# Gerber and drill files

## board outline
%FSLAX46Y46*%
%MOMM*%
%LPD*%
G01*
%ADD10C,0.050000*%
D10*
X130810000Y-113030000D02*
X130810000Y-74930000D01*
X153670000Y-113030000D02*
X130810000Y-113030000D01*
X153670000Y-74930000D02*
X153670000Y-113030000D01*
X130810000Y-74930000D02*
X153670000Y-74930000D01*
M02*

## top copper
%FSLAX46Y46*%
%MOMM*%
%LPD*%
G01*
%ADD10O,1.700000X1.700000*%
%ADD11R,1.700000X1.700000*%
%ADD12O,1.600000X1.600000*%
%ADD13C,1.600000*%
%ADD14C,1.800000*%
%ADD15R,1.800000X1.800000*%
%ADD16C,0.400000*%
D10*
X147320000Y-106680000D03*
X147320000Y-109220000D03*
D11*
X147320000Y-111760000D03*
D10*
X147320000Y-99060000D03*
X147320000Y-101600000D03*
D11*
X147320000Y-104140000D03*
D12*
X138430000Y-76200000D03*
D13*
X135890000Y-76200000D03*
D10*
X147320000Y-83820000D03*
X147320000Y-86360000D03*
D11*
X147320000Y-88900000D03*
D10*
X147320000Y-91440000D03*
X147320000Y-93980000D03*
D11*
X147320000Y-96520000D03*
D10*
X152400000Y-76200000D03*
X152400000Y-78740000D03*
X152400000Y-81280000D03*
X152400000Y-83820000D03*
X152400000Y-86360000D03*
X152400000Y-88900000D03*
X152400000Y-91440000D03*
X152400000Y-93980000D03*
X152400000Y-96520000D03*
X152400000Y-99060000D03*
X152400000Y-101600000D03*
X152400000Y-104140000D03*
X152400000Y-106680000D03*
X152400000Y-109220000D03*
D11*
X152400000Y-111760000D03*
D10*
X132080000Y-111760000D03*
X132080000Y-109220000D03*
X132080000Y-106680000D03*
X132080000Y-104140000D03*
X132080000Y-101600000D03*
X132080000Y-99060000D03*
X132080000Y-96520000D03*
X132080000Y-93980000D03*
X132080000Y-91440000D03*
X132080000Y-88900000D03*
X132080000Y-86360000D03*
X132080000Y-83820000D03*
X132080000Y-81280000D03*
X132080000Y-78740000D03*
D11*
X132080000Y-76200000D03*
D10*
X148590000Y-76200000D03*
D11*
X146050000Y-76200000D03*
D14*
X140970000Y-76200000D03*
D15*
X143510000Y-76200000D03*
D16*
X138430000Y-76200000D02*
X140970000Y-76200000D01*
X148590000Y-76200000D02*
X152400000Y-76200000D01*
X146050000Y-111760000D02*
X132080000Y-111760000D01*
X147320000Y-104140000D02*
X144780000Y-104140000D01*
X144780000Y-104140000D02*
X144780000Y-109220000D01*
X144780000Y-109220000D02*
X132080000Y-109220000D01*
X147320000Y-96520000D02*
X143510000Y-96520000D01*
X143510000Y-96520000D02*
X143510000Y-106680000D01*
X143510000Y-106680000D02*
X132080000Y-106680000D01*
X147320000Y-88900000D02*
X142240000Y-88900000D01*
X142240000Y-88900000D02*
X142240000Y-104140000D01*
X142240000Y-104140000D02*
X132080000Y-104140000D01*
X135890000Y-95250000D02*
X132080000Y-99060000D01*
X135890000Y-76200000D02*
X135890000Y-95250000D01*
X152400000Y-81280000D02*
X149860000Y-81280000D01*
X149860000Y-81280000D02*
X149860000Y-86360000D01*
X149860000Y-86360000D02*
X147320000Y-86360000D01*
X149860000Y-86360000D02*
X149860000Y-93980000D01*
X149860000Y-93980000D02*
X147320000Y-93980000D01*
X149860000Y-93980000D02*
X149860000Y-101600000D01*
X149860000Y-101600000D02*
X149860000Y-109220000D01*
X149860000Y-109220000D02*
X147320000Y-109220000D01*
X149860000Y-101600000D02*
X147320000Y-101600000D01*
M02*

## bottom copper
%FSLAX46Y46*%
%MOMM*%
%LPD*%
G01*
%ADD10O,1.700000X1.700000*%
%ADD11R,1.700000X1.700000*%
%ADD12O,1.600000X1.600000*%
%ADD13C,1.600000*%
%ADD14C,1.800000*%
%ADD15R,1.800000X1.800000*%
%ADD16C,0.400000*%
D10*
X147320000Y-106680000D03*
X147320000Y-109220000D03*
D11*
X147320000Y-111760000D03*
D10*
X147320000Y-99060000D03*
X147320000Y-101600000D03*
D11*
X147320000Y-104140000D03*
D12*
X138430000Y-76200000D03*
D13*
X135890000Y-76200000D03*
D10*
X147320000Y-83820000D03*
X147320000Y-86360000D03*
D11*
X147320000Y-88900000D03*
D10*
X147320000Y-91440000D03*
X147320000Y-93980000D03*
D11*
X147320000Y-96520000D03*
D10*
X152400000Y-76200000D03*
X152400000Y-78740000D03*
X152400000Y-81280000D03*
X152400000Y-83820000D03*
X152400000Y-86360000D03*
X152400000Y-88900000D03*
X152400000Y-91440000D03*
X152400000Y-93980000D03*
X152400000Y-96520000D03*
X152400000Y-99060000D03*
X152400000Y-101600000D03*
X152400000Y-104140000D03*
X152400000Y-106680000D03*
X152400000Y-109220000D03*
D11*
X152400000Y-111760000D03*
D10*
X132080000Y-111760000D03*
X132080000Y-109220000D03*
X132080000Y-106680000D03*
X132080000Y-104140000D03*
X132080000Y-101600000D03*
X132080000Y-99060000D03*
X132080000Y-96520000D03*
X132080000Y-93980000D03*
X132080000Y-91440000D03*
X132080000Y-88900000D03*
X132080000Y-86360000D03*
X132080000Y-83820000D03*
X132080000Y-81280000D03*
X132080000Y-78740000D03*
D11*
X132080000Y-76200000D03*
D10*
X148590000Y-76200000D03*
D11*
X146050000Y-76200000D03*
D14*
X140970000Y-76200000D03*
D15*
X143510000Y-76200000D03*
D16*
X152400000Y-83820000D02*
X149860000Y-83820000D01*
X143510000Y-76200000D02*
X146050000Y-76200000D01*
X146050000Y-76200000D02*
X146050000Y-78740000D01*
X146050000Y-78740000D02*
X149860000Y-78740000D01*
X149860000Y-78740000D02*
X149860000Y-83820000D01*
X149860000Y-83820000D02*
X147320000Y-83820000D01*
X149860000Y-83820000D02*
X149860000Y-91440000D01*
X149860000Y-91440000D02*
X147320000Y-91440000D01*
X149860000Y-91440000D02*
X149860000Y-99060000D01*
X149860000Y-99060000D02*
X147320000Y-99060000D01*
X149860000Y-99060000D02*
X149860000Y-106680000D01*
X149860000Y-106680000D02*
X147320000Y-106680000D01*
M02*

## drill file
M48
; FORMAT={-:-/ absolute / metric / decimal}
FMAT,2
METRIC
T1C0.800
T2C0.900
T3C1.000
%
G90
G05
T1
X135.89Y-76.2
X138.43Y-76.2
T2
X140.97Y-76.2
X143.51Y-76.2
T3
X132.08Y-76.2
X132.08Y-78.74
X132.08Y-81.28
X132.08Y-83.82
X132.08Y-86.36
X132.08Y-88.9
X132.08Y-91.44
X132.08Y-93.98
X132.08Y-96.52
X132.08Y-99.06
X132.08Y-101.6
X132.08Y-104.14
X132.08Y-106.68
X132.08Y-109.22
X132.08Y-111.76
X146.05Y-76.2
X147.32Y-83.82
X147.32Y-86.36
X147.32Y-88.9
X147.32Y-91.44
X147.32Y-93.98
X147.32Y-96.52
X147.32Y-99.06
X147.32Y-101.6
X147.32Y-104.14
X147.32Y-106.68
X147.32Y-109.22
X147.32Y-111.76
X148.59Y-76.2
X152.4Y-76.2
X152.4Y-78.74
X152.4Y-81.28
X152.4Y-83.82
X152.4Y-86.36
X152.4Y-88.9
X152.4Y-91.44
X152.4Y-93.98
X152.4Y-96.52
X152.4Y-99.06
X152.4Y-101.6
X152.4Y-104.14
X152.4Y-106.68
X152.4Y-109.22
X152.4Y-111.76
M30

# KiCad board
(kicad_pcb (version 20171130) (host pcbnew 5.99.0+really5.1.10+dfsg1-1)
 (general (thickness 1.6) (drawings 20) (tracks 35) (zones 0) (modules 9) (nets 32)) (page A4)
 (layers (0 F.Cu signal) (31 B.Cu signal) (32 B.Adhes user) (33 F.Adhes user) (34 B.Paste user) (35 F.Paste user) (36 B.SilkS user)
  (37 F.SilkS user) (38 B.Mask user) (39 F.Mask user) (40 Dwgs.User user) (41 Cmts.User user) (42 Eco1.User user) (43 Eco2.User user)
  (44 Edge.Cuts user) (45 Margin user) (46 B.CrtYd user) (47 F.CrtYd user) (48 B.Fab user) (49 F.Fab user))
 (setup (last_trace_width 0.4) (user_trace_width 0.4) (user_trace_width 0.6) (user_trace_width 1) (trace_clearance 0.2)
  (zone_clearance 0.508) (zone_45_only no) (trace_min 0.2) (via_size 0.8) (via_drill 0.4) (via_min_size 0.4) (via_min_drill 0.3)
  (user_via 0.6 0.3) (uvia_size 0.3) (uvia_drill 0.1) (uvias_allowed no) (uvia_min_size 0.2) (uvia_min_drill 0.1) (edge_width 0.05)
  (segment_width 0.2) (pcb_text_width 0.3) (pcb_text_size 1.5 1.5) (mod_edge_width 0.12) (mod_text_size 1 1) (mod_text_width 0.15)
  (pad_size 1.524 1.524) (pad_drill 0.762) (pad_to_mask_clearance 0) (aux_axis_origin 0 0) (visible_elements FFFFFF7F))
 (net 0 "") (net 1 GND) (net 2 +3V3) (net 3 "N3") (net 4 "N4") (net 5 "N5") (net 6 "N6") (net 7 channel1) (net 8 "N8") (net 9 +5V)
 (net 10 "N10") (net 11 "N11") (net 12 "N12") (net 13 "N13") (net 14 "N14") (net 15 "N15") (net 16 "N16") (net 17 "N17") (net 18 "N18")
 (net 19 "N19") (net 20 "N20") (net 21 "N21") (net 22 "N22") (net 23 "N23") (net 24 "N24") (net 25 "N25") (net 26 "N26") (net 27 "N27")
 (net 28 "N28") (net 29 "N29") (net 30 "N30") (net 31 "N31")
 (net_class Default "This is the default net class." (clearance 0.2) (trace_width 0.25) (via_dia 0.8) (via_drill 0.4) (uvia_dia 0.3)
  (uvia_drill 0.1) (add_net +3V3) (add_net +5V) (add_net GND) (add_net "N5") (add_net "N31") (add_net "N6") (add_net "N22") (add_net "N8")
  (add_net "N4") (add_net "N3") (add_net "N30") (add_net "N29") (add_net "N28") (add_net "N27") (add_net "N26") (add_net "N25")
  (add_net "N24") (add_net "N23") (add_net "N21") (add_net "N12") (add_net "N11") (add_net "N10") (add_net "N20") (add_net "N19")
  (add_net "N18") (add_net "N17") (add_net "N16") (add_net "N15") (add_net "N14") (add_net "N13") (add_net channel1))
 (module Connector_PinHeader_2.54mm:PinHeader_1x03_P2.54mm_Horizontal (layer F.Cu) (at 147.32 111.76 180)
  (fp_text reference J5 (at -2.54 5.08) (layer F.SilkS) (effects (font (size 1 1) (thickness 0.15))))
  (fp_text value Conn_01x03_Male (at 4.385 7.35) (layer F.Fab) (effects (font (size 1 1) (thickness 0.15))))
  (pad 3 thru_hole oval (at 0 5.08 180) (size 1.7 1.7) (drill 1) (layers *.Cu *.Mask) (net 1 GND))
  (pad 2 thru_hole oval (at 0 2.54 180) (size 1.7 1.7) (drill 1) (layers *.Cu *.Mask) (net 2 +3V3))
  (pad 1 thru_hole rect (at 0 0 180) (size 1.7 1.7) (drill 1) (layers *.Cu *.Mask) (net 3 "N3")))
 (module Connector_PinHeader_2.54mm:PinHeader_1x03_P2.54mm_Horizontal (layer F.Cu) (at 147.32 104.14 180)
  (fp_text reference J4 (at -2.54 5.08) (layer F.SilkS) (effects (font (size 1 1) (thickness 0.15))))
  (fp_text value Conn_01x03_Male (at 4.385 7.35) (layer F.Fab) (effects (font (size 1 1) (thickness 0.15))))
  (pad 3 thru_hole oval (at 0 5.08 180) (size 1.7 1.7) (drill 1) (layers *.Cu *.Mask) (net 1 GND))
  (pad 2 thru_hole oval (at 0 2.54 180) (size 1.7 1.7) (drill 1) (layers *.Cu *.Mask) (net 2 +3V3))
  (pad 1 thru_hole rect (at 0 0 180) (size 1.7 1.7) (drill 1) (layers *.Cu *.Mask) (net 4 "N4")))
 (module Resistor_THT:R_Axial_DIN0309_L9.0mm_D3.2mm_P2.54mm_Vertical (layer F.Cu) (at 135.89 76.2)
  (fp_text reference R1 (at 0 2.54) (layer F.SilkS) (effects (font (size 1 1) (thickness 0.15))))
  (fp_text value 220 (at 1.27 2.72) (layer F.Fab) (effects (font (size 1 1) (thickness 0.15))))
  (pad 2 thru_hole oval (at 2.54 0) (size 1.6 1.6) (drill 0.8) (layers *.Cu *.Mask) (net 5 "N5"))
  (pad 1 thru_hole circle (at 0 0) (size 1.6 1.6) (drill 0.8) (layers *.Cu *.Mask) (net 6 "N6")))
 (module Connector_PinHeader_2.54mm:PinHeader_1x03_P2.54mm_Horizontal (layer F.Cu) (at 147.32 88.9 180)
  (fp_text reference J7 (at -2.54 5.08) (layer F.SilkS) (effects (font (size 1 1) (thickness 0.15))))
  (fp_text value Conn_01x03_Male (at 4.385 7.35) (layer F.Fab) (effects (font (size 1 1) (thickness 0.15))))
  (pad 3 thru_hole oval (at 0 5.08 180) (size 1.7 1.7) (drill 1) (layers *.Cu *.Mask) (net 1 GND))
  (pad 2 thru_hole oval (at 0 2.54 180) (size 1.7 1.7) (drill 1) (layers *.Cu *.Mask) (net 2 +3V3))
  (pad 1 thru_hole rect (at 0 0 180) (size 1.7 1.7) (drill 1) (layers *.Cu *.Mask) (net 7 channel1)))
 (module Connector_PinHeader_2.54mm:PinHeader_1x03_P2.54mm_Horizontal (layer F.Cu) (at 147.32 96.52 180)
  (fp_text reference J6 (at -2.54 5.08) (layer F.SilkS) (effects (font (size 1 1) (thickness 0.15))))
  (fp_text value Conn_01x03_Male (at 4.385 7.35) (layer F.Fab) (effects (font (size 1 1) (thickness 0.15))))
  (pad 3 thru_hole oval (at 0 5.08 180) (size 1.7 1.7) (drill 1) (layers *.Cu *.Mask) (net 1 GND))
  (pad 2 thru_hole oval (at 0 2.54 180) (size 1.7 1.7) (drill 1) (layers *.Cu *.Mask) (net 2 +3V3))
  (pad 1 thru_hole rect (at 0 0 180) (size 1.7 1.7) (drill 1) (layers *.Cu *.Mask) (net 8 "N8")))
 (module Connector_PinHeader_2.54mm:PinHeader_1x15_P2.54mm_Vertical (layer F.Cu) (at 152.4 111.76 180)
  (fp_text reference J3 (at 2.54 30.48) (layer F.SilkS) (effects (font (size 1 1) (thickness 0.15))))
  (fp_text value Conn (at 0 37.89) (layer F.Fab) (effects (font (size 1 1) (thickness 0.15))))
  (pad 15 thru_hole oval (at 0 35.56 180) (size 1.7 1.7) (drill 1) (layers *.Cu *.Mask) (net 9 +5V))
  (pad 14 thru_hole oval (at 0 33.02 180) (size 1.7 1.7) (drill 1) (layers *.Cu *.Mask) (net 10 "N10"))
  (pad 13 thru_hole oval (at 0 30.48 180) (size 1.7 1.7) (drill 1) (layers *.Cu *.Mask) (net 2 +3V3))
  (pad 12 thru_hole oval (at 0 27.94 180) (size 1.7 1.7) (drill 1) (layers *.Cu *.Mask) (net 1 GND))
  (pad 11 thru_hole oval (at 0 25.4 180) (size 1.7 1.7) (drill 1) (layers *.Cu *.Mask) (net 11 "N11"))
  (pad 10 thru_hole oval (at 0 22.86 180) (size 1.7 1.7) (drill 1) (layers *.Cu *.Mask) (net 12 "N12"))
  (pad 9 thru_hole oval (at 0 20.32 180) (size 1.7 1.7) (drill 1) (layers *.Cu *.Mask) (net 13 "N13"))
  (pad 8 thru_hole oval (at 0 17.78 180) (size 1.7 1.7) (drill 1) (layers *.Cu *.Mask) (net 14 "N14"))
  (pad 7 thru_hole oval (at 0 15.24 180) (size 1.7 1.7) (drill 1) (layers *.Cu *.Mask) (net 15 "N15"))
  (pad 6 thru_hole oval (at 0 12.7 180) (size 1.7 1.7) (drill 1) (layers *.Cu *.Mask) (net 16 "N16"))
  (pad 5 thru_hole oval (at 0 10.16 180) (size 1.7 1.7) (drill 1) (layers *.Cu *.Mask) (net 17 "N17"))
  (pad 4 thru_hole oval (at 0 7.62 180) (size 1.7 1.7) (drill 1) (layers *.Cu *.Mask) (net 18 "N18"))
  (pad 3 thru_hole oval (at 0 5.08 180) (size 1.7 1.7) (drill 1) (layers *.Cu *.Mask) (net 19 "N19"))
  (pad 2 thru_hole oval (at 0 2.54 180) (size 1.7 1.7) (drill 1) (layers *.Cu *.Mask) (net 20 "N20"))
  (pad 1 thru_hole rect (at 0 0 180) (size 1.7 1.7) (drill 1) (layers *.Cu *.Mask) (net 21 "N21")))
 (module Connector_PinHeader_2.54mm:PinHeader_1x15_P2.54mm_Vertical (layer F.Cu) (at 132.08 76.2)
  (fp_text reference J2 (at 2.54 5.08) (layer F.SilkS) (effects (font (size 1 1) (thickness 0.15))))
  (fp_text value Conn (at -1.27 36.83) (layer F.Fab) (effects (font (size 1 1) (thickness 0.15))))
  (pad 15 thru_hole oval (at 0 35.56) (size 1.7 1.7) (drill 1) (layers *.Cu *.Mask) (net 3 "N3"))
  (pad 14 thru_hole oval (at 0 33.02) (size 1.7 1.7) (drill 1) (layers *.Cu *.Mask) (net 4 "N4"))
  (pad 13 thru_hole oval (at 0 30.48) (size 1.7 1.7) (drill 1) (layers *.Cu *.Mask) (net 8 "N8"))
  (pad 12 thru_hole oval (at 0 27.94) (size 1.7 1.7) (drill 1) (layers *.Cu *.Mask) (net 7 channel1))
  (pad 11 thru_hole oval (at 0 25.4) (size 1.7 1.7) (drill 1) (layers *.Cu *.Mask) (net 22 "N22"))
  (pad 10 thru_hole oval (at 0 22.86) (size 1.7 1.7) (drill 1) (layers *.Cu *.Mask) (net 6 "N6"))
  (pad 9 thru_hole oval (at 0 20.32) (size 1.7 1.7) (drill 1) (layers *.Cu *.Mask) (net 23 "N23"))
  (pad 8 thru_hole oval (at 0 17.78) (size 1.7 1.7) (drill 1) (layers *.Cu *.Mask) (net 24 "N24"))
  (pad 7 thru_hole oval (at 0 15.24) (size 1.7 1.7) (drill 1) (layers *.Cu *.Mask) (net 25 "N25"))
  (pad 6 thru_hole oval (at 0 12.7) (size 1.7 1.7) (drill 1) (layers *.Cu *.Mask) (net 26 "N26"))
  (pad 5 thru_hole oval (at 0 10.16) (size 1.7 1.7) (drill 1) (layers *.Cu *.Mask) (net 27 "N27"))
  (pad 4 thru_hole oval (at 0 7.62) (size 1.7 1.7) (drill 1) (layers *.Cu *.Mask) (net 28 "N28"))
  (pad 3 thru_hole oval (at 0 5.08) (size 1.7 1.7) (drill 1) (layers *.Cu *.Mask) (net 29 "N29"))
  (pad 2 thru_hole oval (at 0 2.54) (size 1.7 1.7) (drill 1) (layers *.Cu *.Mask) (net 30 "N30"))
  (pad 1 thru_hole rect (at 0 0) (size 1.7 1.7) (drill 1) (layers *.Cu *.Mask) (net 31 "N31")))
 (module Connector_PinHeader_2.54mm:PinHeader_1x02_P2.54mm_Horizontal (layer F.Cu) (at 146.05 76.2 90)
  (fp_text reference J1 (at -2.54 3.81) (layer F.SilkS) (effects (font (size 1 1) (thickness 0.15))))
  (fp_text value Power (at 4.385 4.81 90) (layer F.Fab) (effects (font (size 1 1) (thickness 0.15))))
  (pad 2 thru_hole oval (at 0 2.54 90) (size 1.7 1.7) (drill 1) (layers *.Cu *.Mask) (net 9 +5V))
  (pad 1 thru_hole rect (at 0 0 90) (size 1.7 1.7) (drill 1) (layers *.Cu *.Mask) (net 1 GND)))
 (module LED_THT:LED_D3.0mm (layer F.Cu) (at 143.51 76.2 180)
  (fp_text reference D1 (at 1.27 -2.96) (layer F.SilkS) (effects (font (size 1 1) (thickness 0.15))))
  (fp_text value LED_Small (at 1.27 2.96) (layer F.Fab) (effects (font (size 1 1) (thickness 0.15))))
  (pad 2 thru_hole circle (at 2.54 0 180) (size 1.8 1.8) (drill 0.9) (layers *.Cu *.Mask) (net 5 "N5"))
  (pad 1 thru_hole rect (at 0 0 180) (size 1.8 1.8) (drill 0.9) (layers *.Cu *.Mask) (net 1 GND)))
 (gr_line (start 130.81 113.03) (end 130.81 74.93) (layer Edge.Cuts) (width 0.05))
 (gr_line (start 153.67 113.03) (end 130.81 113.03) (layer Edge.Cuts) (width 0.05))
 (gr_line (start 153.67 74.93) (end 153.67 113.03) (layer Edge.Cuts) (width 0.05))
 (gr_line (start 130.81 74.93) (end 153.67 74.93) (layer Edge.Cuts) (width 0.05))
 (segment (start 138.43 76.2) (end 140.97 76.2) (width 0.4) (layer F.Cu) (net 5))
 (segment (start 152.4 83.82) (end 149.86 83.82) (width 0.4) (layer B.Cu) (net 1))
 (segment (start 143.51 76.2) (end 146.05 76.2) (width 0.4) (layer B.Cu) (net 1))
 (segment (start 146.05 76.2) (end 146.05 78.74) (width 0.4) (layer B.Cu) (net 1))
 (segment (start 146.05 78.74) (end 149.86 78.74) (width 0.4) (layer B.Cu) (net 1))
 (segment (start 149.86 78.74) (end 149.86 83.82) (width 0.4) (layer B.Cu) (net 1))
 (segment (start 149.86 83.82) (end 147.32 83.82) (width 0.4) (layer B.Cu) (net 1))
 (segment (start 149.86 83.82) (end 149.86 91.44) (width 0.4) (layer B.Cu) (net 1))
 (segment (start 149.86 91.44) (end 147.32 91.44) (width 0.4) (layer B.Cu) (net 1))
 (segment (start 149.86 91.44) (end 149.86 99.06) (width 0.4) (layer B.Cu) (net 1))
 (segment (start 149.86 99.06) (end 147.32 99.06) (width 0.4) (layer B.Cu) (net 1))
 (segment (start 149.86 99.06) (end 149.86 106.68) (width 0.4) (layer B.Cu) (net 1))
 (segment (start 149.86 106.68) (end 147.32 106.68) (width 0.4) (layer B.Cu) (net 1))
 (segment (start 148.59 76.2) (end 152.4 76.2) (width 0.4) (layer F.Cu) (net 9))
 (segment (start 146.05 111.76) (end 132.08 111.76) (width 0.4) (layer F.Cu) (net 3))
 (segment (start 147.32 104.14) (end 144.78 104.14) (width 0.4) (layer F.Cu) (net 4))
 (segment (start 144.78 104.14) (end 144.78 109.22) (width 0.4) (layer F.Cu) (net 4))
 (segment (start 144.78 109.22) (end 132.08 109.22) (width 0.4) (layer F.Cu) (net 4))
 (segment (start 147.32 96.52) (end 143.51 96.52) (width 0.4) (layer F.Cu) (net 8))
 (segment (start 143.51 96.52) (end 143.51 106.68) (width 0.4) (layer F.Cu) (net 8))
 (segment (start 143.51 106.68) (end 132.08 106.68) (width 0.4) (layer F.Cu) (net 8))
 (segment (start 147.32 88.9) (end 142.24 88.9) (width 0.4) (layer F.Cu) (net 7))
 (segment (start 142.24 88.9) (end 142.24 104.14) (width 0.4) (layer F.Cu) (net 7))
 (segment (start 142.24 104.14) (end 132.08 104.14) (width 0.4) (layer F.Cu) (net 7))
 (segment (start 135.89 95.25) (end 132.08 99.06) (width 0.4) (layer F.Cu) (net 6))
 (segment (start 135.89 76.2) (end 135.89 95.25) (width 0.4) (layer F.Cu) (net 6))
 (segment (start 152.4 81.28) (end 149.86 81.28) (width 0.4) (layer F.Cu) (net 2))
 (segment (start 149.86 81.28) (end 149.86 86.36) (width 0.4) (layer F.Cu) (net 2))
 (segment (start 149.86 86.36) (end 147.32 86.36) (width 0.4) (layer F.Cu) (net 2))
 (segment (start 149.86 86.36) (end 149.86 93.98) (width 0.4) (layer F.Cu) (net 2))
 (segment (start 149.86 93.98) (end 147.32 93.98) (width 0.4) (layer F.Cu) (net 2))
 (segment (start 149.86 93.98) (end 149.86 101.6) (width 0.4) (layer F.Cu) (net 2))
 (segment (start 149.86 101.6) (end 149.86 109.22) (width 0.4) (layer F.Cu) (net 2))
 (segment (start 149.86 109.22) (end 147.32 109.22) (width 0.4) (layer F.Cu) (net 2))
 (segment (start 149.86 101.6) (end 147.32 101.6) (width 0.4) (layer F.Cu) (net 2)))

